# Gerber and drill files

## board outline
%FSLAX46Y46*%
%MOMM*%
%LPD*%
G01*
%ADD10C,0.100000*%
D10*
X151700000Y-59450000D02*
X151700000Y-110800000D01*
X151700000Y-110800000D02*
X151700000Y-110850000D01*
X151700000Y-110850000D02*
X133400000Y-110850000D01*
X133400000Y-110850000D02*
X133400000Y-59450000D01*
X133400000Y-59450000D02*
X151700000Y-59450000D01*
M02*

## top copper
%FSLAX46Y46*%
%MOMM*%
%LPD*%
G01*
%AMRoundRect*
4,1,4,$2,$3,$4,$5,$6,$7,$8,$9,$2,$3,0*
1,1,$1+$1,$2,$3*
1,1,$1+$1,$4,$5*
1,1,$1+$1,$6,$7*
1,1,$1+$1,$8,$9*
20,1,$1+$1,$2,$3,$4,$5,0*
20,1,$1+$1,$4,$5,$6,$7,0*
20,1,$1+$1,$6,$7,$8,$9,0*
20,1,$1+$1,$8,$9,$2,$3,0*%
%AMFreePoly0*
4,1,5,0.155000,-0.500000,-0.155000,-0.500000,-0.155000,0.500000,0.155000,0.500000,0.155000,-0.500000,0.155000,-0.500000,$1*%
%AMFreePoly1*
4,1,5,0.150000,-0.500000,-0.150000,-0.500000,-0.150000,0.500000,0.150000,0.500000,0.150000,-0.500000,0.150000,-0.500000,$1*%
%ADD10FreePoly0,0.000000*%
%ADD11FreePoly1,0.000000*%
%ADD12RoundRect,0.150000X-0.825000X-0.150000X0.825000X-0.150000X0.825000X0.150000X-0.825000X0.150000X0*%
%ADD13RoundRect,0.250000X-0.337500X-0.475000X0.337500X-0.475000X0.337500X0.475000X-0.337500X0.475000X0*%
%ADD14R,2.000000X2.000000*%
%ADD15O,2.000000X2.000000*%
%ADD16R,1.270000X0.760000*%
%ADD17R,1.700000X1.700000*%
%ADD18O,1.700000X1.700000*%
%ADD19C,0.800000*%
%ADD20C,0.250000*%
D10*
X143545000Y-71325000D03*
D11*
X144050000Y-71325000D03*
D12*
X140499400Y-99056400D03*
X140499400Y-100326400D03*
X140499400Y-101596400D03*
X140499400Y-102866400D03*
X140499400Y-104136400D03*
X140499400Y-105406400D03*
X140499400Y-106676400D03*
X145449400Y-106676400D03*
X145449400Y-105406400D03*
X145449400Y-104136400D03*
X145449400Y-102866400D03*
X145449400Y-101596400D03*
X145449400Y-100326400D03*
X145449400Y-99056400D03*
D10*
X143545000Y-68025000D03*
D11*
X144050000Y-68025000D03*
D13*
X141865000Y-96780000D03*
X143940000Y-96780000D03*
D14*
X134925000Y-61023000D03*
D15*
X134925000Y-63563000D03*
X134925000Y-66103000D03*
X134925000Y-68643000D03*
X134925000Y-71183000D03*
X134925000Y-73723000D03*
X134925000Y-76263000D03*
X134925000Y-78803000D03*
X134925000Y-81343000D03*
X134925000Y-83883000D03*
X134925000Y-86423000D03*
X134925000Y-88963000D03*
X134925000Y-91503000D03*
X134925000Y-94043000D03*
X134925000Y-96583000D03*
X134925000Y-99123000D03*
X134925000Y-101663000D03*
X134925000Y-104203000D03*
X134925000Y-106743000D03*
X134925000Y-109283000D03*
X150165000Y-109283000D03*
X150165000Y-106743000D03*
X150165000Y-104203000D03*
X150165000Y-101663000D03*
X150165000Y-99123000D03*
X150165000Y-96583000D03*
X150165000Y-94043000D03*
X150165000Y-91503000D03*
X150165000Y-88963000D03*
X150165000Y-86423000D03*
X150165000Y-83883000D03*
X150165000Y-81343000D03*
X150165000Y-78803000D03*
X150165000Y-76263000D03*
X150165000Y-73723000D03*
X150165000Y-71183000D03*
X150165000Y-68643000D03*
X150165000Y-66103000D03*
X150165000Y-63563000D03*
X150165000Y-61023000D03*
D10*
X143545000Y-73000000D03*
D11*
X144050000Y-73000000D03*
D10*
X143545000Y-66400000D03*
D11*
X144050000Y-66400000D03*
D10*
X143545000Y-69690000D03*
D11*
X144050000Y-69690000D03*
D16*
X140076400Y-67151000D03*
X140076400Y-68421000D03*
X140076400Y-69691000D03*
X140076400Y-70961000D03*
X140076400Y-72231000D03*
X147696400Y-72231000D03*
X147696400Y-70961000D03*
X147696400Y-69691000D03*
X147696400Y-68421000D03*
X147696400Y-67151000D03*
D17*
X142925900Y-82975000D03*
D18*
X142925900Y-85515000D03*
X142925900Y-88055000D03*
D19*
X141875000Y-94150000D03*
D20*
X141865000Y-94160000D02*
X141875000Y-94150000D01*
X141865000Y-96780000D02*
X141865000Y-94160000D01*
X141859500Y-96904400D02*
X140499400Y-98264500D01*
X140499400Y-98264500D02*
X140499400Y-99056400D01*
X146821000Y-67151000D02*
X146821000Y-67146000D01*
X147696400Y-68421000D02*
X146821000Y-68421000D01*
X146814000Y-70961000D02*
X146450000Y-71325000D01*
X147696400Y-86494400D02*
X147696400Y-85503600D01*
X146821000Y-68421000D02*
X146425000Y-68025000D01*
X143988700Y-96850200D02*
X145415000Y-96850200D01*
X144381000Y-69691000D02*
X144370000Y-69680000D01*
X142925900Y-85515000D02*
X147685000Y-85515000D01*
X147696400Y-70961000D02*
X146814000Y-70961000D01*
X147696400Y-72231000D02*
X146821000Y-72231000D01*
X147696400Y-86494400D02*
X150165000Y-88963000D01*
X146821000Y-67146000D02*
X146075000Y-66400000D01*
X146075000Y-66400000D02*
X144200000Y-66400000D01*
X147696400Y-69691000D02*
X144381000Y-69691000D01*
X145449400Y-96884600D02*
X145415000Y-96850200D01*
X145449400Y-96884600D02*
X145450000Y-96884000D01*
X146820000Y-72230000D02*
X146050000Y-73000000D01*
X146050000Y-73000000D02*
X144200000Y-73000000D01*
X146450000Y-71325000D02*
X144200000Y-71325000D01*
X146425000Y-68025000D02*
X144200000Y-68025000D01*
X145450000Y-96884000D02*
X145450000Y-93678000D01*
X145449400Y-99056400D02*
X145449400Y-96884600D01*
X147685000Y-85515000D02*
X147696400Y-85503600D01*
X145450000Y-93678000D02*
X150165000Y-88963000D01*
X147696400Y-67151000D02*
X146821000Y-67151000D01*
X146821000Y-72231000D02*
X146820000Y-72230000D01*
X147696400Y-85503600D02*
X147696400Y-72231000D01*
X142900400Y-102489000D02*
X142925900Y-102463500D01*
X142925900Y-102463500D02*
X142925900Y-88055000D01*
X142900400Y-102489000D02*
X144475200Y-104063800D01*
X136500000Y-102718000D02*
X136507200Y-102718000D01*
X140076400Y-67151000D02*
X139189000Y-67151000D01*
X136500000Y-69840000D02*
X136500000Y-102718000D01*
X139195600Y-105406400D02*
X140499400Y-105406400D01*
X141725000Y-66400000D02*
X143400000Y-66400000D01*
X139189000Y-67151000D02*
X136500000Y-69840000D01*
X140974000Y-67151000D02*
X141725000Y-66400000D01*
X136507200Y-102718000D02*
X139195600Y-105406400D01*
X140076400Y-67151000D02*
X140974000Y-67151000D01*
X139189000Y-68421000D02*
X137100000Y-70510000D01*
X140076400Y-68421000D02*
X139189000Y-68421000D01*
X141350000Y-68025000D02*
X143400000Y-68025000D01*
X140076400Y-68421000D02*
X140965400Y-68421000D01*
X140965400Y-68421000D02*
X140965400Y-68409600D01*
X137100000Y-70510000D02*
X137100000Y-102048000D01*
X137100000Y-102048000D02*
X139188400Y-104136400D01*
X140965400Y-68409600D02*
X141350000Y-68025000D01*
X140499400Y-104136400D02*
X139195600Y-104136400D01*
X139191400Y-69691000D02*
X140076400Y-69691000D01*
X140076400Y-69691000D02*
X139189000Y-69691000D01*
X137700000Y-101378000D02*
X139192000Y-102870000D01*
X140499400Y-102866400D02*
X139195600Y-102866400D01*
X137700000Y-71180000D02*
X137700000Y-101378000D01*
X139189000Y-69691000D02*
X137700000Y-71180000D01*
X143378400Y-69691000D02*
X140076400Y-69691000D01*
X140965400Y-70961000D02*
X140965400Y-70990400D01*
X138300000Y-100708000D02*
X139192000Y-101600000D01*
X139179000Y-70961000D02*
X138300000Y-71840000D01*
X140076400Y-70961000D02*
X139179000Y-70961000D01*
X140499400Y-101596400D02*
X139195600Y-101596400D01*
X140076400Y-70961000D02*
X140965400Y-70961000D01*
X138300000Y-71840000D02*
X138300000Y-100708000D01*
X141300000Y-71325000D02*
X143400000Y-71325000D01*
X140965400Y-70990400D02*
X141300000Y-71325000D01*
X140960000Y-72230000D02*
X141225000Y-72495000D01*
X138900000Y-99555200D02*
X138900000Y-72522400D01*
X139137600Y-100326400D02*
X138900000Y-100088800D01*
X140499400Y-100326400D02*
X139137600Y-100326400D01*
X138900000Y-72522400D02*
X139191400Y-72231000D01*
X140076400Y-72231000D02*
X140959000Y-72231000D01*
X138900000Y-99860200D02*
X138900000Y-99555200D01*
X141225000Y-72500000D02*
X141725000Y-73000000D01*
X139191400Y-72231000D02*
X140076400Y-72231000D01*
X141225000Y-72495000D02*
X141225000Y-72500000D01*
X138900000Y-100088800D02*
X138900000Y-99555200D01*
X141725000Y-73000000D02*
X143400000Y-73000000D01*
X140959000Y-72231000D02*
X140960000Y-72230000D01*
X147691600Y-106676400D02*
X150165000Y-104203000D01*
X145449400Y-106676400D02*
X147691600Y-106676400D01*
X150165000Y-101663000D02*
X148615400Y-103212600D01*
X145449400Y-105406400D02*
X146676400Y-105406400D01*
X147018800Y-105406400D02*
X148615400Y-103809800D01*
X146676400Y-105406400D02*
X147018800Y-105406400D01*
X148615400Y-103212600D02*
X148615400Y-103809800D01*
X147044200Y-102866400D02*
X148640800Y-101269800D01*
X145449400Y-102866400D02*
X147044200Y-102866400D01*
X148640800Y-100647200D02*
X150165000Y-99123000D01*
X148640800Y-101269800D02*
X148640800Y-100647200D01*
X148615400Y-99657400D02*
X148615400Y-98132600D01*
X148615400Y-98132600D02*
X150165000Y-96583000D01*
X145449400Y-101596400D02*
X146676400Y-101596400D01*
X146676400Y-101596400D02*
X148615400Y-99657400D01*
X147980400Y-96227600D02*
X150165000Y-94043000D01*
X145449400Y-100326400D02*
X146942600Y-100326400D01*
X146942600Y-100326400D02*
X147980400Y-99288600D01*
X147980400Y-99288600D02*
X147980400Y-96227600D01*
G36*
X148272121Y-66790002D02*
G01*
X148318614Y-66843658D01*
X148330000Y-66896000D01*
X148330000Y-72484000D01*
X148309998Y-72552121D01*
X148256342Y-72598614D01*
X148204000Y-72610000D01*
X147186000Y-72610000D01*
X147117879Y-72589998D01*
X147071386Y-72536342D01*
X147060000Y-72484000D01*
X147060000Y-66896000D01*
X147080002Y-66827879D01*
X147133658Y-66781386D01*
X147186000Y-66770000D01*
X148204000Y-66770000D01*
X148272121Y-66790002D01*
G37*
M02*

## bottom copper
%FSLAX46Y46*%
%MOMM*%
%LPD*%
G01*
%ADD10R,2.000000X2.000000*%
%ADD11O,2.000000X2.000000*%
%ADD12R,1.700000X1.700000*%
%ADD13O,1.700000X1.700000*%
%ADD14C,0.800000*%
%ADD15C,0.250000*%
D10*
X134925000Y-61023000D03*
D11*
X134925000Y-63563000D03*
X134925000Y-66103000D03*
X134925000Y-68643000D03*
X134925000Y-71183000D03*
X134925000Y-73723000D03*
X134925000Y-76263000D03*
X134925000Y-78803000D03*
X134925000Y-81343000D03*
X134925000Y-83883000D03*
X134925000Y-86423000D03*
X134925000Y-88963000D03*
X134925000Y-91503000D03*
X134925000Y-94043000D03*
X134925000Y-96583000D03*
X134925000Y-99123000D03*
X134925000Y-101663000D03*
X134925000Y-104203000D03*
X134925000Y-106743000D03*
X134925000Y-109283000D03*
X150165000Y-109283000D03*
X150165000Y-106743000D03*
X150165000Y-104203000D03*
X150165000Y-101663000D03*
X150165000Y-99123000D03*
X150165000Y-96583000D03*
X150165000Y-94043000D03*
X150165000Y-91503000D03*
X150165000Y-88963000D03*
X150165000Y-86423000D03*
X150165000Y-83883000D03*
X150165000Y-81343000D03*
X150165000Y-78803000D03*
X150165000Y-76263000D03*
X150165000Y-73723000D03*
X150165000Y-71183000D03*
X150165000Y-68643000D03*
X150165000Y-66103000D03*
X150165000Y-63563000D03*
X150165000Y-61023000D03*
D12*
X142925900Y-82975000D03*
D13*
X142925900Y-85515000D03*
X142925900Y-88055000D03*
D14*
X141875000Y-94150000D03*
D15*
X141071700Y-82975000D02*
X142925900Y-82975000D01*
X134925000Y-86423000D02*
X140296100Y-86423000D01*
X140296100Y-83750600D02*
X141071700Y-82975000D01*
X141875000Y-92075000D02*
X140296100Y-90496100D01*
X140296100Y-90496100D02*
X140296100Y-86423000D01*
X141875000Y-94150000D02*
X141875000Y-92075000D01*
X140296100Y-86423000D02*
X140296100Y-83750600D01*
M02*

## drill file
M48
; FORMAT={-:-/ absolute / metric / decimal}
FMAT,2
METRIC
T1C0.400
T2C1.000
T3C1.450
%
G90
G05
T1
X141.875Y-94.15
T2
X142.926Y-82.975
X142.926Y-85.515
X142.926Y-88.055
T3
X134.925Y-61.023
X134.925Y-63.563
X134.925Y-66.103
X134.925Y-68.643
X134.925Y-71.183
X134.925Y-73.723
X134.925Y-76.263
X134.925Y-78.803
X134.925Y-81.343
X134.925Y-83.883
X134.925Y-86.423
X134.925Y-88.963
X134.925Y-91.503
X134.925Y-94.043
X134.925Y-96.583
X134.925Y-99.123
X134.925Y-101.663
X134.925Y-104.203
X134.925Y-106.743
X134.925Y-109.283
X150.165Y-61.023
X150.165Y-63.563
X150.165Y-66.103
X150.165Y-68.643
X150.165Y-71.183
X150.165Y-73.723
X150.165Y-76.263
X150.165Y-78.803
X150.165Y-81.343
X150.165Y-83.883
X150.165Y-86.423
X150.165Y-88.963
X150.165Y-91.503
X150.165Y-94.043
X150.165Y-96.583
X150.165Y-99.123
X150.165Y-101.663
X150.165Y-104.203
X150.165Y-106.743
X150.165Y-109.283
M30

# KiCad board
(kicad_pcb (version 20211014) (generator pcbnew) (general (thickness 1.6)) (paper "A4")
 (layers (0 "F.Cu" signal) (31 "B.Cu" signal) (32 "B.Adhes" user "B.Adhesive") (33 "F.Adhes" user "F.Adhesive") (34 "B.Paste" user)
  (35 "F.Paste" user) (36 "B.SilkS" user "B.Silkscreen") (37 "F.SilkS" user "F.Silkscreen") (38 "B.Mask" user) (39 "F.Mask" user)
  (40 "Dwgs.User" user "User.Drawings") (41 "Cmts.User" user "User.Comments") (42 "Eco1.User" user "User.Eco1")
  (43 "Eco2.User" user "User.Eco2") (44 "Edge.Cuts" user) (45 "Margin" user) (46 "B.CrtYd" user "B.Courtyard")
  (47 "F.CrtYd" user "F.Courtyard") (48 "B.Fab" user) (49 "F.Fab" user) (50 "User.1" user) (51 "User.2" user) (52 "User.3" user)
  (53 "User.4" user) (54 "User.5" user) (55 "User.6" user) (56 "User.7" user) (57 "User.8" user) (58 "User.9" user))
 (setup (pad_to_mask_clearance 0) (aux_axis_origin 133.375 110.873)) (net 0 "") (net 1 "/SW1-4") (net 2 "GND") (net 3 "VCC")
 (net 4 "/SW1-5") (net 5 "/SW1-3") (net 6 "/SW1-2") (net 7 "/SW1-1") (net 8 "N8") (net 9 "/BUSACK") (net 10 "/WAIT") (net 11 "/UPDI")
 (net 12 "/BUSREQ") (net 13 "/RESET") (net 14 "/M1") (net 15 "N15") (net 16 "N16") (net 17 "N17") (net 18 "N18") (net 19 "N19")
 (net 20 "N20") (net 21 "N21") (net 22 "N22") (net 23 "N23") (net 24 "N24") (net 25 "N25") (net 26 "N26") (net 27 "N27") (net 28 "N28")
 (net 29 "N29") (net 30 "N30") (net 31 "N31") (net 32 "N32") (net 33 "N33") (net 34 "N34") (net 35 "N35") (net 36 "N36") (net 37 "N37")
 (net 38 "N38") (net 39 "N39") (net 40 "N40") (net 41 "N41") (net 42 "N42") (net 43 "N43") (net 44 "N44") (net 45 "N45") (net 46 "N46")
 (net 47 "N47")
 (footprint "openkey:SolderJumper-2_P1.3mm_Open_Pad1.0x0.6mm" (layer "F.Cu") (at 143.8 71.325)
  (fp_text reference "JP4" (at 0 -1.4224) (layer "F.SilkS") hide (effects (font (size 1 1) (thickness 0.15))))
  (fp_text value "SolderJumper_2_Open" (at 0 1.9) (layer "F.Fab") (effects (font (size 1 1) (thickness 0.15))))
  (pad "1" smd custom (at -0.255 0) (size 0.31 1) (layers "F.Cu" "F.Mask") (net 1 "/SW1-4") (options (clearance outline) (anchor rect))
   (primitives))
  (pad "2" smd custom (at 0.25 0) (size 0.3 1) (layers "F.Cu" "F.Mask") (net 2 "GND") (options (clearance outline) (anchor rect))
   (primitives)))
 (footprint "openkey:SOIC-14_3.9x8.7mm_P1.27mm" (layer "F.Cu") (at 142.9744 102.8664)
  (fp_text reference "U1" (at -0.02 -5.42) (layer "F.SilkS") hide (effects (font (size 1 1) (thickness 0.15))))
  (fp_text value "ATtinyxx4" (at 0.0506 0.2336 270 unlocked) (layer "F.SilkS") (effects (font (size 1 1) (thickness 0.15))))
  (pad "1" smd roundrect (at -2.475 -3.81) (size 1.95 0.6) (layers "F.Cu" "F.Paste" "F.Mask") (roundrect_rratio 0.25) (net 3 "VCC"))
  (pad "2" smd roundrect (at -2.475 -2.54) (size 1.95 0.6) (layers "F.Cu" "F.Paste" "F.Mask") (roundrect_rratio 0.25) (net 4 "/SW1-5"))
  (pad "3" smd roundrect (at -2.475 -1.27) (size 1.95 0.6) (layers "F.Cu" "F.Paste" "F.Mask") (roundrect_rratio 0.25) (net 1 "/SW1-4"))
  (pad "4" smd roundrect (at -2.475 0) (size 1.95 0.6) (layers "F.Cu" "F.Paste" "F.Mask") (roundrect_rratio 0.25) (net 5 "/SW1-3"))
  (pad "5" smd roundrect (at -2.475 1.27) (size 1.95 0.6) (layers "F.Cu" "F.Paste" "F.Mask") (roundrect_rratio 0.25) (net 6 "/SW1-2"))
  (pad "6" smd roundrect (at -2.475 2.54) (size 1.95 0.6) (layers "F.Cu" "F.Paste" "F.Mask") (roundrect_rratio 0.25) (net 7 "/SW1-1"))
  (pad "7" smd roundrect (at -2.475 3.81) (size 1.95 0.6) (layers "F.Cu" "F.Paste" "F.Mask") (roundrect_rratio 0.25) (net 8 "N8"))
  (pad "8" smd roundrect (at 2.475 3.81) (size 1.95 0.6) (layers "F.Cu" "F.Paste" "F.Mask") (roundrect_rratio 0.25) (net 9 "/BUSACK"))
  (pad "9" smd roundrect (at 2.475 2.54) (size 1.95 0.6) (layers "F.Cu" "F.Paste" "F.Mask") (roundrect_rratio 0.25) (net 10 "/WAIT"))
  (pad "10" smd roundrect (at 2.475 1.27) (size 1.95 0.6) (layers "F.Cu" "F.Paste" "F.Mask") (roundrect_rratio 0.25) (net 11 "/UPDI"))
  (pad "11" smd roundrect (at 2.475 0) (size 1.95 0.6) (layers "F.Cu" "F.Paste" "F.Mask") (roundrect_rratio 0.25) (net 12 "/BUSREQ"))
  (pad "12" smd roundrect (at 2.475 -1.27) (size 1.95 0.6) (layers "F.Cu" "F.Paste" "F.Mask") (roundrect_rratio 0.25) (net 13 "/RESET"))
  (pad "13" smd roundrect (at 2.475 -2.54) (size 1.95 0.6) (layers "F.Cu" "F.Paste" "F.Mask") (roundrect_rratio 0.25) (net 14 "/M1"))
  (pad "14" smd roundrect (at 2.475 -3.81) (size 1.95 0.6) (layers "F.Cu" "F.Paste" "F.Mask") (roundrect_rratio 0.25) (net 2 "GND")))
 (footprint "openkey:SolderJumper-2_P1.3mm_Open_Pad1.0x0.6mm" (layer "F.Cu") (at 143.8 68.025)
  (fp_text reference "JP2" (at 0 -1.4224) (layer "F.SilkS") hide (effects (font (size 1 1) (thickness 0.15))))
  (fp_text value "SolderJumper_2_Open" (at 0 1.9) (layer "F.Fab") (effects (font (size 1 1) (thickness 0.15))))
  (pad "1" smd custom (at -0.255 0) (size 0.31 1) (layers "F.Cu" "F.Mask") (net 6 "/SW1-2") (options (clearance outline) (anchor rect))
   (primitives))
  (pad "2" smd custom (at 0.25 0) (size 0.3 1) (layers "F.Cu" "F.Mask") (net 2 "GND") (options (clearance outline) (anchor rect))
   (primitives)))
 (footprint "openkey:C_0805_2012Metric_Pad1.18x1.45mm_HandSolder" (layer "F.Cu") (at 142.9025 96.78)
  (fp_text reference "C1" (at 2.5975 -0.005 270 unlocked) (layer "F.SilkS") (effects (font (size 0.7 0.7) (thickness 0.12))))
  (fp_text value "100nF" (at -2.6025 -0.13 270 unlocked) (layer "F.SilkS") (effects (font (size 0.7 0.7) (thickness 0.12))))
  (pad "1" smd roundrect (at -1.0375 0) (size 1.175 1.45) (layers "F.Cu" "F.Paste" "F.Mask") (roundrect_rratio 0.212766) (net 3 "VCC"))
  (pad "2" smd roundrect (at 1.0375 0) (size 1.175 1.45) (layers "F.Cu" "F.Paste" "F.Mask") (roundrect_rratio 0.212766) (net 2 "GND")))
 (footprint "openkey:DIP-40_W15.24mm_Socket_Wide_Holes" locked (layer "F.Cu") (at 134.925 61.023)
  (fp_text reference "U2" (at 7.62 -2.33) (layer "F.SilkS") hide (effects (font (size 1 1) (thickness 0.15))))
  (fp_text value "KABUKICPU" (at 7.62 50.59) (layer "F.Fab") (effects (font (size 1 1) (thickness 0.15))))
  (pad "1" thru_hole rect locked (at 0 0) (size 2 2) (drill 1.45) (layers *.Cu *.Mask) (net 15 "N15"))
  (pad "2" thru_hole oval locked (at 0 2.54) (size 2 2) (drill 1.45) (layers *.Cu *.Mask) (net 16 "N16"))
  (pad "3" thru_hole oval locked (at 0 5.08) (size 2 2) (drill 1.45) (layers *.Cu *.Mask) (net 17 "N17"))
  (pad "4" thru_hole oval locked (at 0 7.62) (size 2 2) (drill 1.45) (layers *.Cu *.Mask) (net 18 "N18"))
  (pad "5" thru_hole oval locked (at 0 10.16) (size 2 2) (drill 1.45) (layers *.Cu *.Mask) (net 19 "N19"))
  (pad "6" thru_hole oval locked (at 0 12.7) (size 2 2) (drill 1.45) (layers *.Cu *.Mask) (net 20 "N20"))
  (pad "7" thru_hole oval locked (at 0 15.24) (size 2 2) (drill 1.45) (layers *.Cu *.Mask) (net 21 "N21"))
  (pad "8" thru_hole oval locked (at 0 17.78) (size 2 2) (drill 1.45) (layers *.Cu *.Mask) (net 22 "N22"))
  (pad "9" thru_hole oval locked (at 0 20.32) (size 2 2) (drill 1.45) (layers *.Cu *.Mask) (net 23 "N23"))
  (pad "10" thru_hole oval locked (at 0 22.86) (size 2 2) (drill 1.45) (layers *.Cu *.Mask) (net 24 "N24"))
  (pad "11" thru_hole oval locked (at 0 25.4) (size 2 2) (drill 1.45) (layers *.Cu *.Mask) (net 3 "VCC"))
  (pad "12" thru_hole oval locked (at 0 27.94) (size 2 2) (drill 1.45) (layers *.Cu *.Mask) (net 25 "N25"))
  (pad "13" thru_hole oval locked (at 0 30.48) (size 2 2) (drill 1.45) (layers *.Cu *.Mask) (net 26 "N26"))
  (pad "14" thru_hole oval locked (at 0 33.02) (size 2 2) (drill 1.45) (layers *.Cu *.Mask) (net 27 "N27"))
  (pad "15" thru_hole oval locked (at 0 35.56) (size 2 2) (drill 1.45) (layers *.Cu *.Mask) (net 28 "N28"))
  (pad "16" thru_hole oval locked (at 0 38.1) (size 2 2) (drill 1.45) (layers *.Cu *.Mask) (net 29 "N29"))
  (pad "17" thru_hole oval locked (at 0 40.64) (size 2 2) (drill 1.45) (layers *.Cu *.Mask) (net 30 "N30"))
  (pad "18" thru_hole oval locked (at 0 43.18) (size 2 2) (drill 1.45) (layers *.Cu *.Mask) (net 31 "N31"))
  (pad "19" thru_hole oval locked (at 0 45.72) (size 2 2) (drill 1.45) (layers *.Cu *.Mask) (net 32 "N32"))
  (pad "20" thru_hole oval locked (at 0 48.26) (size 2 2) (drill 1.45) (layers *.Cu *.Mask) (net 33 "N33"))
  (pad "21" thru_hole oval locked (at 15.24 48.26) (size 2 2) (drill 1.45) (layers *.Cu *.Mask) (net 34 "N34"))
  (pad "22" thru_hole oval locked (at 15.24 45.72) (size 2 2) (drill 1.45) (layers *.Cu *.Mask) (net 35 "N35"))
  (pad "23" thru_hole oval locked (at 15.24 43.18) (size 2 2) (drill 1.45) (layers *.Cu *.Mask) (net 9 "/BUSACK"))
  (pad "24" thru_hole oval locked (at 15.24 40.64) (size 2 2) (drill 1.45) (layers *.Cu *.Mask) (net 10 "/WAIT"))
  (pad "25" thru_hole oval locked (at 15.24 38.1) (size 2 2) (drill 1.45) (layers *.Cu *.Mask) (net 12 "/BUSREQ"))
  (pad "26" thru_hole oval locked (at 15.24 35.56) (size 2 2) (drill 1.45) (layers *.Cu *.Mask) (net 13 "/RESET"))
  (pad "27" thru_hole oval locked (at 15.24 33.02) (size 2 2) (drill 1.45) (layers *.Cu *.Mask) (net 14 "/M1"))
  (pad "28" thru_hole oval locked (at 15.24 30.48) (size 2 2) (drill 1.45) (layers *.Cu *.Mask) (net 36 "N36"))
  (pad "29" thru_hole oval locked (at 15.24 27.94) (size 2 2) (drill 1.45) (layers *.Cu *.Mask) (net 2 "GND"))
  (pad "30" thru_hole oval locked (at 15.24 25.4) (size 2 2) (drill 1.45) (layers *.Cu *.Mask) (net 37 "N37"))
  (pad "31" thru_hole oval locked (at 15.24 22.86) (size 2 2) (drill 1.45) (layers *.Cu *.Mask) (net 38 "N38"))
  (pad "32" thru_hole oval locked (at 15.24 20.32) (size 2 2) (drill 1.45) (layers *.Cu *.Mask) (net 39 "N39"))
  (pad "33" thru_hole oval locked (at 15.24 17.78) (size 2 2) (drill 1.45) (layers *.Cu *.Mask) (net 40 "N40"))
  (pad "34" thru_hole oval locked (at 15.24 15.24) (size 2 2) (drill 1.45) (layers *.Cu *.Mask) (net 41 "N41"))
  (pad "35" thru_hole oval locked (at 15.24 12.7) (size 2 2) (drill 1.45) (layers *.Cu *.Mask) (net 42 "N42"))
  (pad "36" thru_hole oval locked (at 15.24 10.16) (size 2 2) (drill 1.45) (layers *.Cu *.Mask) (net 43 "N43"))
  (pad "37" thru_hole oval locked (at 15.24 7.62) (size 2 2) (drill 1.45) (layers *.Cu *.Mask) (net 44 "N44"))
  (pad "38" thru_hole oval locked (at 15.24 5.08) (size 2 2) (drill 1.45) (layers *.Cu *.Mask) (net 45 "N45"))
  (pad "39" thru_hole oval locked (at 15.24 2.54) (size 2 2) (drill 1.45) (layers *.Cu *.Mask) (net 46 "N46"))
  (pad "40" thru_hole oval locked (at 15.24 0) (size 2 2) (drill 1.45) (layers *.Cu *.Mask) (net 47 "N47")))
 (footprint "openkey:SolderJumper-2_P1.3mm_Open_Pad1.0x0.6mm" (layer "F.Cu") (at 143.8 73)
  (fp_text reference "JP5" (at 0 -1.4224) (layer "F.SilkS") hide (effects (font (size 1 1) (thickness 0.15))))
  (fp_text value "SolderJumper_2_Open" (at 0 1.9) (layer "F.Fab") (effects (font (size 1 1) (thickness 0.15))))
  (pad "1" smd custom (at -0.255 0) (size 0.31 1) (layers "F.Cu" "F.Mask") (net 4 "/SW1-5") (options (clearance outline) (anchor rect))
   (primitives))
  (pad "2" smd custom (at 0.25 0) (size 0.3 1) (layers "F.Cu" "F.Mask") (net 2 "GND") (options (clearance outline) (anchor rect))
   (primitives)))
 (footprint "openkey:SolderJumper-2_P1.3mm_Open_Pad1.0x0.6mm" (layer "F.Cu") (at 143.8 66.4)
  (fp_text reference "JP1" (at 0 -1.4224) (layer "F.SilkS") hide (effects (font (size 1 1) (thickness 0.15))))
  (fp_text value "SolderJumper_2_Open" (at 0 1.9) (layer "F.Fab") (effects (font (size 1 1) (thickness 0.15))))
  (pad "1" smd custom (at -0.255 0) (size 0.31 1) (layers "F.Cu" "F.Mask") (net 7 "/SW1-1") (options (clearance outline) (anchor rect))
   (primitives))
  (pad "2" smd custom (at 0.25 0) (size 0.3 1) (layers "F.Cu" "F.Mask") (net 2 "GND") (options (clearance outline) (anchor rect))
   (primitives)))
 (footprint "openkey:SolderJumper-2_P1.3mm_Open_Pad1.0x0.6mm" (layer "F.Cu") (at 143.8 69.69)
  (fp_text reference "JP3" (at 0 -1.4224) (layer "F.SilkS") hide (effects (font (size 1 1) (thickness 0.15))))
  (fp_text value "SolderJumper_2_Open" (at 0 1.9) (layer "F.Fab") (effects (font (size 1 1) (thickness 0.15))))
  (pad "1" smd custom (at -0.255 0) (size 0.31 1) (layers "F.Cu" "F.Mask") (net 5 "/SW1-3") (options (clearance outline) (anchor rect))
   (primitives))
  (pad "2" smd custom (at 0.25 0) (size 0.3 1) (layers "F.Cu" "F.Mask") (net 2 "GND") (options (clearance outline) (anchor rect))
   (primitives)))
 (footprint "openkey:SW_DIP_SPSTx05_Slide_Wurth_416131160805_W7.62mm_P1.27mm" (layer "F.Cu") (at 143.8864 69.691)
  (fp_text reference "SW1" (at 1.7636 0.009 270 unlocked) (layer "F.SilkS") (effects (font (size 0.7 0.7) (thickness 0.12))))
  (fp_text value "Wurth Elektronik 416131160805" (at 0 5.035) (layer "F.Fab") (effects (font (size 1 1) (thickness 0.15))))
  (pad "1" smd rect (at -3.81 -2.54) (size 1.27 0.76) (layers "F.Cu" "F.Paste" "F.Mask") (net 7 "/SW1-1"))
  (pad "2" smd rect (at -3.81 -1.27) (size 1.27 0.76) (layers "F.Cu" "F.Paste" "F.Mask") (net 6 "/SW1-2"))
  (pad "3" smd rect (at -3.81 0) (size 1.27 0.76) (layers "F.Cu" "F.Paste" "F.Mask") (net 5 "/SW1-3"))
  (pad "4" smd rect (at -3.81 1.27) (size 1.27 0.76) (layers "F.Cu" "F.Paste" "F.Mask") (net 1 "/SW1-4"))
  (pad "5" smd rect (at -3.81 2.54) (size 1.27 0.76) (layers "F.Cu" "F.Paste" "F.Mask") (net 4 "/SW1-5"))
  (pad "6" smd rect (at 3.81 2.54) (size 1.27 0.76) (layers "F.Cu" "F.Paste" "F.Mask") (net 2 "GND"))
  (pad "7" smd rect (at 3.81 1.27) (size 1.27 0.76) (layers "F.Cu" "F.Paste" "F.Mask") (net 2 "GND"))
  (pad "8" smd rect (at 3.81 0) (size 1.27 0.76) (layers "F.Cu" "F.Paste" "F.Mask") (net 2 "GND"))
  (pad "9" smd rect (at 3.81 -1.27) (size 1.27 0.76) (layers "F.Cu" "F.Paste" "F.Mask") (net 2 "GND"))
  (pad "10" smd rect (at 3.81 -2.54) (size 1.27 0.76) (layers "F.Cu" "F.Paste" "F.Mask") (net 2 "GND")))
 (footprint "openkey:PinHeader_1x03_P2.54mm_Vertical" (layer "F.Cu") (at 142.9259 82.975)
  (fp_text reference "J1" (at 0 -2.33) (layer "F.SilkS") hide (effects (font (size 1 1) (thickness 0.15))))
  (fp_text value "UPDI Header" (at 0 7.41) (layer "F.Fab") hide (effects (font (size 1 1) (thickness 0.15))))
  (pad "1" thru_hole rect (at 0 0) (size 1.7 1.7) (drill 1) (layers *.Cu *.Mask) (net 3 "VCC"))
  (pad "2" thru_hole oval (at 0 2.54) (size 1.7 1.7) (drill 1) (layers *.Cu *.Mask) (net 2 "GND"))
  (pad "3" thru_hole oval (at 0 5.08) (size 1.7 1.7) (drill 1) (layers *.Cu *.Mask) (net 11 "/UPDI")))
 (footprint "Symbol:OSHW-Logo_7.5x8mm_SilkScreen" (layer "B.Cu") (at 142.375 105.6 180)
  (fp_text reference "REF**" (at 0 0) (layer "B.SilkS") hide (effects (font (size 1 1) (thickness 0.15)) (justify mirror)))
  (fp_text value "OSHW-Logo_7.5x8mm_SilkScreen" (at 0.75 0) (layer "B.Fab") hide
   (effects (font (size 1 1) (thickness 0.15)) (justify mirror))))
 (gr_line (start 151.7 59.45) (end 151.7 110.8) (layer "Edge.Cuts") (width 0.1))
 (gr_line (start 151.7 110.8) (end 151.7 110.85) (layer "Edge.Cuts") (width 0.1))
 (gr_line (start 151.7 110.85) (end 133.4 110.85) (layer "Edge.Cuts") (width 0.1))
 (gr_line (start 133.4 110.85) (end 133.4 59.45) (layer "Edge.Cuts") (width 0.1))
 (gr_line (start 133.4 59.45) (end 151.7 59.45) (layer "Edge.Cuts") (width 0.1))
 (segment (start 141.865 94.16) (end 141.875 94.15) (width 0.25) (layer "F.Cu") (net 3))
 (segment (start 141.865 96.78) (end 141.865 94.16) (width 0.25) (layer "F.Cu") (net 3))
 (segment (start 141.8595 96.9044) (end 140.4994 98.2645) (width 0.25) (layer "F.Cu") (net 3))
 (segment (start 140.4994 98.2645) (end 140.4994 99.0564) (width 0.25) (layer "F.Cu") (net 3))
 (via (at 141.875 94.15) (size 0.8) (drill 0.4) (layers "F.Cu" "B.Cu") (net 3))
 (segment (start 141.0717 82.975) (end 142.9259 82.975) (width 0.25) (layer "B.Cu") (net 3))
 (segment (start 134.925 86.423) (end 140.2961 86.423) (width 0.25) (layer "B.Cu") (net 3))
 (segment (start 140.2961 83.7506) (end 141.0717 82.975) (width 0.25) (layer "B.Cu") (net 3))
 (segment (start 141.875 92.075) (end 140.2961 90.4961) (width 0.25) (layer "B.Cu") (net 3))
 (segment (start 140.2961 90.4961) (end 140.2961 86.423) (width 0.25) (layer "B.Cu") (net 3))
 (segment (start 141.875 94.15) (end 141.875 92.075) (width 0.25) (layer "B.Cu") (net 3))
 (segment (start 140.2961 86.423) (end 140.2961 83.7506) (width 0.25) (layer "B.Cu") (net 3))
 (segment (start 146.821 67.151) (end 146.821 67.146) (width 0.25) (layer "F.Cu") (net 2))
 (segment (start 147.6964 68.421) (end 146.821 68.421) (width 0.25) (layer "F.Cu") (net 2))
 (segment (start 146.814 70.961) (end 146.45 71.325) (width 0.25) (layer "F.Cu") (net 2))
 (segment (start 147.6964 86.4944) (end 147.6964 85.5036) (width 0.25) (layer "F.Cu") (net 2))
 (segment (start 146.821 68.421) (end 146.425 68.025) (width 0.25) (layer "F.Cu") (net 2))
 (segment (start 143.9887 96.8502) (end 145.415 96.8502) (width 0.25) (layer "F.Cu") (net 2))
 (segment (start 144.381 69.691) (end 144.37 69.68) (width 0.25) (layer "F.Cu") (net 2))
 (segment (start 142.9259 85.515) (end 147.685 85.515) (width 0.25) (layer "F.Cu") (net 2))
 (segment (start 147.6964 70.961) (end 146.814 70.961) (width 0.25) (layer "F.Cu") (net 2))
 (segment (start 147.6964 72.231) (end 146.821 72.231) (width 0.25) (layer "F.Cu") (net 2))
 (segment (start 147.6964 86.4944) (end 150.165 88.963) (width 0.25) (layer "F.Cu") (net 2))
 (segment (start 146.821 67.146) (end 146.075 66.4) (width 0.25) (layer "F.Cu") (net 2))
 (segment (start 146.075 66.4) (end 144.2 66.4) (width 0.25) (layer "F.Cu") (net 2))
 (segment (start 147.6964 69.691) (end 144.381 69.691) (width 0.25) (layer "F.Cu") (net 2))
 (segment (start 145.4494 96.8846) (end 145.415 96.8502) (width 0.25) (layer "F.Cu") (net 2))
 (segment (start 145.4494 96.8846) (end 145.45 96.884) (width 0.25) (layer "F.Cu") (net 2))
 (segment (start 146.82 72.23) (end 146.05 73) (width 0.25) (layer "F.Cu") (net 2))
 (segment (start 146.05 73) (end 144.2 73) (width 0.25) (layer "F.Cu") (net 2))
 (segment (start 146.45 71.325) (end 144.2 71.325) (width 0.25) (layer "F.Cu") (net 2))
 (segment (start 146.425 68.025) (end 144.2 68.025) (width 0.25) (layer "F.Cu") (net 2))
 (segment (start 145.45 96.884) (end 145.45 93.678) (width 0.25) (layer "F.Cu") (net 2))
 (segment (start 145.4494 99.0564) (end 145.4494 96.8846) (width 0.25) (layer "F.Cu") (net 2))
 (segment (start 147.685 85.515) (end 147.6964 85.5036) (width 0.25) (layer "F.Cu") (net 2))
 (segment (start 145.45 93.678) (end 150.165 88.963) (width 0.25) (layer "F.Cu") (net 2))
 (segment (start 147.6964 67.151) (end 146.821 67.151) (width 0.25) (layer "F.Cu") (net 2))
 (segment (start 146.821 72.231) (end 146.82 72.23) (width 0.25) (layer "F.Cu") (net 2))
 (segment (start 147.6964 85.5036) (end 147.6964 72.231) (width 0.25) (layer "F.Cu") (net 2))
 (segment (start 142.9004 102.489) (end 142.9259 102.4635) (width 0.25) (layer "F.Cu") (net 11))
 (segment (start 142.9259 102.4635) (end 142.9259 88.055) (width 0.25) (layer "F.Cu") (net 11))
 (segment (start 142.9004 102.489) (end 144.4752 104.0638) (width 0.25) (layer "F.Cu") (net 11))
 (segment (start 136.5 102.718) (end 136.5072 102.718) (width 0.25) (layer "F.Cu") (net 7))
 (segment (start 140.0764 67.151) (end 139.189 67.151) (width 0.25) (layer "F.Cu") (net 7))
 (segment (start 136.5 69.84) (end 136.5 102.718) (width 0.25) (layer "F.Cu") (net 7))
 (segment (start 139.1956 105.4064) (end 140.4994 105.4064) (width 0.25) (layer "F.Cu") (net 7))
 (segment (start 141.725 66.4) (end 143.4 66.4) (width 0.25) (layer "F.Cu") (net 7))
 (segment (start 139.189 67.151) (end 136.5 69.84) (width 0.25) (layer "F.Cu") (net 7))
 (segment (start 140.974 67.151) (end 141.725 66.4) (width 0.25) (layer "F.Cu") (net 7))
 (segment (start 136.5072 102.718) (end 139.1956 105.4064) (width 0.25) (layer "F.Cu") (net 7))
 (segment (start 140.0764 67.151) (end 140.974 67.151) (width 0.25) (layer "F.Cu") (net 7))
 (segment (start 139.189 68.421) (end 137.1 70.51) (width 0.25) (layer "F.Cu") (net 6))
 (segment (start 140.0764 68.421) (end 139.189 68.421) (width 0.25) (layer "F.Cu") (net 6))
 (segment (start 141.35 68.025) (end 143.4 68.025) (width 0.25) (layer "F.Cu") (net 6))
 (segment (start 140.0764 68.421) (end 140.9654 68.421) (width 0.25) (layer "F.Cu") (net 6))
 (segment (start 140.9654 68.421) (end 140.9654 68.4096) (width 0.25) (layer "F.Cu") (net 6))
 (segment (start 137.1 70.51) (end 137.1 102.048) (width 0.25) (layer "F.Cu") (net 6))
 (segment (start 137.1 102.048) (end 139.1884 104.1364) (width 0.25) (layer "F.Cu") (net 6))
 (segment (start 140.9654 68.4096) (end 141.35 68.025) (width 0.25) (layer "F.Cu") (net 6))
 (segment (start 140.4994 104.1364) (end 139.1956 104.1364) (width 0.25) (layer "F.Cu") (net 6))
 (segment (start 139.1914 69.691) (end 140.0764 69.691) (width 0.25) (layer "F.Cu") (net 5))
 (segment (start 140.0764 69.691) (end 139.189 69.691) (width 0.25) (layer "F.Cu") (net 5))
 (segment (start 137.7 101.378) (end 139.192 102.87) (width 0.25) (layer "F.Cu") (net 5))
 (segment (start 140.4994 102.8664) (end 139.1956 102.8664) (width 0.25) (layer "F.Cu") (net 5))
 (segment (start 137.7 71.18) (end 137.7 101.378) (width 0.25) (layer "F.Cu") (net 5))
 (segment (start 139.189 69.691) (end 137.7 71.18) (width 0.25) (layer "F.Cu") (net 5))
 (segment (start 143.3784 69.691) (end 140.0764 69.691) (width 0.25) (layer "F.Cu") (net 5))
 (segment (start 140.9654 70.961) (end 140.9654 70.9904) (width 0.25) (layer "F.Cu") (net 1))
 (segment (start 138.3 100.708) (end 139.192 101.6) (width 0.25) (layer "F.Cu") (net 1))
 (segment (start 139.179 70.961) (end 138.3 71.84) (width 0.25) (layer "F.Cu") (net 1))
 (segment (start 140.0764 70.961) (end 139.179 70.961) (width 0.25) (layer "F.Cu") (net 1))
 (segment (start 140.4994 101.5964) (end 139.1956 101.5964) (width 0.25) (layer "F.Cu") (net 1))
 (segment (start 140.0764 70.961) (end 140.9654 70.961) (width 0.25) (layer "F.Cu") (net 1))
 (segment (start 138.3 71.84) (end 138.3 100.708) (width 0.25) (layer "F.Cu") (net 1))
 (segment (start 141.3 71.325) (end 143.4 71.325) (width 0.25) (layer "F.Cu") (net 1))
 (segment (start 140.9654 70.9904) (end 141.3 71.325) (width 0.25) (layer "F.Cu") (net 1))
 (segment (start 140.96 72.23) (end 141.225 72.495) (width 0.25) (layer "F.Cu") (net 4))
 (segment (start 138.9 99.5552) (end 138.9 72.5224) (width 0.25) (layer "F.Cu") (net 4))
 (segment (start 139.1376 100.3264) (end 138.9 100.0888) (width 0.25) (layer "F.Cu") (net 4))
 (segment (start 140.4994 100.3264) (end 139.1376 100.3264) (width 0.25) (layer "F.Cu") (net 4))
 (segment (start 138.9 72.5224) (end 139.1914 72.231) (width 0.25) (layer "F.Cu") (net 4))
 (segment (start 140.0764 72.231) (end 140.959 72.231) (width 0.25) (layer "F.Cu") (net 4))
 (segment (start 138.9 99.8602) (end 138.9 99.5552) (width 0.25) (layer "F.Cu") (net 4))
 (segment (start 141.225 72.5) (end 141.725 73) (width 0.25) (layer "F.Cu") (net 4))
 (segment (start 139.1914 72.231) (end 140.0764 72.231) (width 0.25) (layer "F.Cu") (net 4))
 (segment (start 141.225 72.495) (end 141.225 72.5) (width 0.25) (layer "F.Cu") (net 4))
 (segment (start 138.9 100.0888) (end 138.9 99.5552) (width 0.25) (layer "F.Cu") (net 4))
 (segment (start 141.725 73) (end 143.4 73) (width 0.25) (layer "F.Cu") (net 4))
 (segment (start 140.959 72.231) (end 140.96 72.23) (width 0.25) (layer "F.Cu") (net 4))
 (segment (start 147.6916 106.6764) (end 150.165 104.203) (width 0.25) (layer "F.Cu") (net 9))
 (segment (start 145.4494 106.6764) (end 147.6916 106.6764) (width 0.25) (layer "F.Cu") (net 9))
 (segment (start 150.165 101.663) (end 148.6154 103.2126) (width 0.25) (layer "F.Cu") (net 10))
 (segment (start 145.4494 105.4064) (end 146.6764 105.4064) (width 0.25) (layer "F.Cu") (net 10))
 (segment (start 147.0188 105.4064) (end 148.6154 103.8098) (width 0.25) (layer "F.Cu") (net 10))
 (segment (start 146.6764 105.4064) (end 147.0188 105.4064) (width 0.25) (layer "F.Cu") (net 10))
 (segment (start 148.6154 103.2126) (end 148.6154 103.8098) (width 0.25) (layer "F.Cu") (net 10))
 (segment (start 147.0442 102.8664) (end 148.6408 101.2698) (width 0.25) (layer "F.Cu") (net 12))
 (segment (start 145.4494 102.8664) (end 147.0442 102.8664) (width 0.25) (layer "F.Cu") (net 12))
 (segment (start 148.6408 100.6472) (end 150.165 99.123) (width 0.25) (layer "F.Cu") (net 12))
 (segment (start 148.6408 101.2698) (end 148.6408 100.6472) (width 0.25) (layer "F.Cu") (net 12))
 (segment (start 148.6154 99.6574) (end 148.6154 98.1326) (width 0.25) (layer "F.Cu") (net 13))
 (segment (start 148.6154 98.1326) (end 150.165 96.583) (width 0.25) (layer "F.Cu") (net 13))
 (segment (start 145.4494 101.5964) (end 146.6764 101.5964) (width 0.25) (layer "F.Cu") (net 13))
 (segment (start 146.6764 101.5964) (end 148.6154 99.6574) (width 0.25) (layer "F.Cu") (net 13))
 (segment (start 147.9804 96.2276) (end 150.165 94.043) (width 0.25) (layer "F.Cu") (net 14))
 (segment (start 145.4494 100.3264) (end 146.9426 100.3264) (width 0.25) (layer "F.Cu") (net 14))
 (segment (start 146.9426 100.3264) (end 147.9804 99.2886) (width 0.25) (layer "F.Cu") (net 14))
 (segment (start 147.9804 99.2886) (end 147.9804 96.2276) (width 0.25) (layer "F.Cu") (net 14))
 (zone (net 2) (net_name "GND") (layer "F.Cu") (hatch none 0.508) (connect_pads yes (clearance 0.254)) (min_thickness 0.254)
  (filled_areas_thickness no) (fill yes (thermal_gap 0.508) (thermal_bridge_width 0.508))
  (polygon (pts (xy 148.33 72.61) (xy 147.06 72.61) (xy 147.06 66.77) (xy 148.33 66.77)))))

